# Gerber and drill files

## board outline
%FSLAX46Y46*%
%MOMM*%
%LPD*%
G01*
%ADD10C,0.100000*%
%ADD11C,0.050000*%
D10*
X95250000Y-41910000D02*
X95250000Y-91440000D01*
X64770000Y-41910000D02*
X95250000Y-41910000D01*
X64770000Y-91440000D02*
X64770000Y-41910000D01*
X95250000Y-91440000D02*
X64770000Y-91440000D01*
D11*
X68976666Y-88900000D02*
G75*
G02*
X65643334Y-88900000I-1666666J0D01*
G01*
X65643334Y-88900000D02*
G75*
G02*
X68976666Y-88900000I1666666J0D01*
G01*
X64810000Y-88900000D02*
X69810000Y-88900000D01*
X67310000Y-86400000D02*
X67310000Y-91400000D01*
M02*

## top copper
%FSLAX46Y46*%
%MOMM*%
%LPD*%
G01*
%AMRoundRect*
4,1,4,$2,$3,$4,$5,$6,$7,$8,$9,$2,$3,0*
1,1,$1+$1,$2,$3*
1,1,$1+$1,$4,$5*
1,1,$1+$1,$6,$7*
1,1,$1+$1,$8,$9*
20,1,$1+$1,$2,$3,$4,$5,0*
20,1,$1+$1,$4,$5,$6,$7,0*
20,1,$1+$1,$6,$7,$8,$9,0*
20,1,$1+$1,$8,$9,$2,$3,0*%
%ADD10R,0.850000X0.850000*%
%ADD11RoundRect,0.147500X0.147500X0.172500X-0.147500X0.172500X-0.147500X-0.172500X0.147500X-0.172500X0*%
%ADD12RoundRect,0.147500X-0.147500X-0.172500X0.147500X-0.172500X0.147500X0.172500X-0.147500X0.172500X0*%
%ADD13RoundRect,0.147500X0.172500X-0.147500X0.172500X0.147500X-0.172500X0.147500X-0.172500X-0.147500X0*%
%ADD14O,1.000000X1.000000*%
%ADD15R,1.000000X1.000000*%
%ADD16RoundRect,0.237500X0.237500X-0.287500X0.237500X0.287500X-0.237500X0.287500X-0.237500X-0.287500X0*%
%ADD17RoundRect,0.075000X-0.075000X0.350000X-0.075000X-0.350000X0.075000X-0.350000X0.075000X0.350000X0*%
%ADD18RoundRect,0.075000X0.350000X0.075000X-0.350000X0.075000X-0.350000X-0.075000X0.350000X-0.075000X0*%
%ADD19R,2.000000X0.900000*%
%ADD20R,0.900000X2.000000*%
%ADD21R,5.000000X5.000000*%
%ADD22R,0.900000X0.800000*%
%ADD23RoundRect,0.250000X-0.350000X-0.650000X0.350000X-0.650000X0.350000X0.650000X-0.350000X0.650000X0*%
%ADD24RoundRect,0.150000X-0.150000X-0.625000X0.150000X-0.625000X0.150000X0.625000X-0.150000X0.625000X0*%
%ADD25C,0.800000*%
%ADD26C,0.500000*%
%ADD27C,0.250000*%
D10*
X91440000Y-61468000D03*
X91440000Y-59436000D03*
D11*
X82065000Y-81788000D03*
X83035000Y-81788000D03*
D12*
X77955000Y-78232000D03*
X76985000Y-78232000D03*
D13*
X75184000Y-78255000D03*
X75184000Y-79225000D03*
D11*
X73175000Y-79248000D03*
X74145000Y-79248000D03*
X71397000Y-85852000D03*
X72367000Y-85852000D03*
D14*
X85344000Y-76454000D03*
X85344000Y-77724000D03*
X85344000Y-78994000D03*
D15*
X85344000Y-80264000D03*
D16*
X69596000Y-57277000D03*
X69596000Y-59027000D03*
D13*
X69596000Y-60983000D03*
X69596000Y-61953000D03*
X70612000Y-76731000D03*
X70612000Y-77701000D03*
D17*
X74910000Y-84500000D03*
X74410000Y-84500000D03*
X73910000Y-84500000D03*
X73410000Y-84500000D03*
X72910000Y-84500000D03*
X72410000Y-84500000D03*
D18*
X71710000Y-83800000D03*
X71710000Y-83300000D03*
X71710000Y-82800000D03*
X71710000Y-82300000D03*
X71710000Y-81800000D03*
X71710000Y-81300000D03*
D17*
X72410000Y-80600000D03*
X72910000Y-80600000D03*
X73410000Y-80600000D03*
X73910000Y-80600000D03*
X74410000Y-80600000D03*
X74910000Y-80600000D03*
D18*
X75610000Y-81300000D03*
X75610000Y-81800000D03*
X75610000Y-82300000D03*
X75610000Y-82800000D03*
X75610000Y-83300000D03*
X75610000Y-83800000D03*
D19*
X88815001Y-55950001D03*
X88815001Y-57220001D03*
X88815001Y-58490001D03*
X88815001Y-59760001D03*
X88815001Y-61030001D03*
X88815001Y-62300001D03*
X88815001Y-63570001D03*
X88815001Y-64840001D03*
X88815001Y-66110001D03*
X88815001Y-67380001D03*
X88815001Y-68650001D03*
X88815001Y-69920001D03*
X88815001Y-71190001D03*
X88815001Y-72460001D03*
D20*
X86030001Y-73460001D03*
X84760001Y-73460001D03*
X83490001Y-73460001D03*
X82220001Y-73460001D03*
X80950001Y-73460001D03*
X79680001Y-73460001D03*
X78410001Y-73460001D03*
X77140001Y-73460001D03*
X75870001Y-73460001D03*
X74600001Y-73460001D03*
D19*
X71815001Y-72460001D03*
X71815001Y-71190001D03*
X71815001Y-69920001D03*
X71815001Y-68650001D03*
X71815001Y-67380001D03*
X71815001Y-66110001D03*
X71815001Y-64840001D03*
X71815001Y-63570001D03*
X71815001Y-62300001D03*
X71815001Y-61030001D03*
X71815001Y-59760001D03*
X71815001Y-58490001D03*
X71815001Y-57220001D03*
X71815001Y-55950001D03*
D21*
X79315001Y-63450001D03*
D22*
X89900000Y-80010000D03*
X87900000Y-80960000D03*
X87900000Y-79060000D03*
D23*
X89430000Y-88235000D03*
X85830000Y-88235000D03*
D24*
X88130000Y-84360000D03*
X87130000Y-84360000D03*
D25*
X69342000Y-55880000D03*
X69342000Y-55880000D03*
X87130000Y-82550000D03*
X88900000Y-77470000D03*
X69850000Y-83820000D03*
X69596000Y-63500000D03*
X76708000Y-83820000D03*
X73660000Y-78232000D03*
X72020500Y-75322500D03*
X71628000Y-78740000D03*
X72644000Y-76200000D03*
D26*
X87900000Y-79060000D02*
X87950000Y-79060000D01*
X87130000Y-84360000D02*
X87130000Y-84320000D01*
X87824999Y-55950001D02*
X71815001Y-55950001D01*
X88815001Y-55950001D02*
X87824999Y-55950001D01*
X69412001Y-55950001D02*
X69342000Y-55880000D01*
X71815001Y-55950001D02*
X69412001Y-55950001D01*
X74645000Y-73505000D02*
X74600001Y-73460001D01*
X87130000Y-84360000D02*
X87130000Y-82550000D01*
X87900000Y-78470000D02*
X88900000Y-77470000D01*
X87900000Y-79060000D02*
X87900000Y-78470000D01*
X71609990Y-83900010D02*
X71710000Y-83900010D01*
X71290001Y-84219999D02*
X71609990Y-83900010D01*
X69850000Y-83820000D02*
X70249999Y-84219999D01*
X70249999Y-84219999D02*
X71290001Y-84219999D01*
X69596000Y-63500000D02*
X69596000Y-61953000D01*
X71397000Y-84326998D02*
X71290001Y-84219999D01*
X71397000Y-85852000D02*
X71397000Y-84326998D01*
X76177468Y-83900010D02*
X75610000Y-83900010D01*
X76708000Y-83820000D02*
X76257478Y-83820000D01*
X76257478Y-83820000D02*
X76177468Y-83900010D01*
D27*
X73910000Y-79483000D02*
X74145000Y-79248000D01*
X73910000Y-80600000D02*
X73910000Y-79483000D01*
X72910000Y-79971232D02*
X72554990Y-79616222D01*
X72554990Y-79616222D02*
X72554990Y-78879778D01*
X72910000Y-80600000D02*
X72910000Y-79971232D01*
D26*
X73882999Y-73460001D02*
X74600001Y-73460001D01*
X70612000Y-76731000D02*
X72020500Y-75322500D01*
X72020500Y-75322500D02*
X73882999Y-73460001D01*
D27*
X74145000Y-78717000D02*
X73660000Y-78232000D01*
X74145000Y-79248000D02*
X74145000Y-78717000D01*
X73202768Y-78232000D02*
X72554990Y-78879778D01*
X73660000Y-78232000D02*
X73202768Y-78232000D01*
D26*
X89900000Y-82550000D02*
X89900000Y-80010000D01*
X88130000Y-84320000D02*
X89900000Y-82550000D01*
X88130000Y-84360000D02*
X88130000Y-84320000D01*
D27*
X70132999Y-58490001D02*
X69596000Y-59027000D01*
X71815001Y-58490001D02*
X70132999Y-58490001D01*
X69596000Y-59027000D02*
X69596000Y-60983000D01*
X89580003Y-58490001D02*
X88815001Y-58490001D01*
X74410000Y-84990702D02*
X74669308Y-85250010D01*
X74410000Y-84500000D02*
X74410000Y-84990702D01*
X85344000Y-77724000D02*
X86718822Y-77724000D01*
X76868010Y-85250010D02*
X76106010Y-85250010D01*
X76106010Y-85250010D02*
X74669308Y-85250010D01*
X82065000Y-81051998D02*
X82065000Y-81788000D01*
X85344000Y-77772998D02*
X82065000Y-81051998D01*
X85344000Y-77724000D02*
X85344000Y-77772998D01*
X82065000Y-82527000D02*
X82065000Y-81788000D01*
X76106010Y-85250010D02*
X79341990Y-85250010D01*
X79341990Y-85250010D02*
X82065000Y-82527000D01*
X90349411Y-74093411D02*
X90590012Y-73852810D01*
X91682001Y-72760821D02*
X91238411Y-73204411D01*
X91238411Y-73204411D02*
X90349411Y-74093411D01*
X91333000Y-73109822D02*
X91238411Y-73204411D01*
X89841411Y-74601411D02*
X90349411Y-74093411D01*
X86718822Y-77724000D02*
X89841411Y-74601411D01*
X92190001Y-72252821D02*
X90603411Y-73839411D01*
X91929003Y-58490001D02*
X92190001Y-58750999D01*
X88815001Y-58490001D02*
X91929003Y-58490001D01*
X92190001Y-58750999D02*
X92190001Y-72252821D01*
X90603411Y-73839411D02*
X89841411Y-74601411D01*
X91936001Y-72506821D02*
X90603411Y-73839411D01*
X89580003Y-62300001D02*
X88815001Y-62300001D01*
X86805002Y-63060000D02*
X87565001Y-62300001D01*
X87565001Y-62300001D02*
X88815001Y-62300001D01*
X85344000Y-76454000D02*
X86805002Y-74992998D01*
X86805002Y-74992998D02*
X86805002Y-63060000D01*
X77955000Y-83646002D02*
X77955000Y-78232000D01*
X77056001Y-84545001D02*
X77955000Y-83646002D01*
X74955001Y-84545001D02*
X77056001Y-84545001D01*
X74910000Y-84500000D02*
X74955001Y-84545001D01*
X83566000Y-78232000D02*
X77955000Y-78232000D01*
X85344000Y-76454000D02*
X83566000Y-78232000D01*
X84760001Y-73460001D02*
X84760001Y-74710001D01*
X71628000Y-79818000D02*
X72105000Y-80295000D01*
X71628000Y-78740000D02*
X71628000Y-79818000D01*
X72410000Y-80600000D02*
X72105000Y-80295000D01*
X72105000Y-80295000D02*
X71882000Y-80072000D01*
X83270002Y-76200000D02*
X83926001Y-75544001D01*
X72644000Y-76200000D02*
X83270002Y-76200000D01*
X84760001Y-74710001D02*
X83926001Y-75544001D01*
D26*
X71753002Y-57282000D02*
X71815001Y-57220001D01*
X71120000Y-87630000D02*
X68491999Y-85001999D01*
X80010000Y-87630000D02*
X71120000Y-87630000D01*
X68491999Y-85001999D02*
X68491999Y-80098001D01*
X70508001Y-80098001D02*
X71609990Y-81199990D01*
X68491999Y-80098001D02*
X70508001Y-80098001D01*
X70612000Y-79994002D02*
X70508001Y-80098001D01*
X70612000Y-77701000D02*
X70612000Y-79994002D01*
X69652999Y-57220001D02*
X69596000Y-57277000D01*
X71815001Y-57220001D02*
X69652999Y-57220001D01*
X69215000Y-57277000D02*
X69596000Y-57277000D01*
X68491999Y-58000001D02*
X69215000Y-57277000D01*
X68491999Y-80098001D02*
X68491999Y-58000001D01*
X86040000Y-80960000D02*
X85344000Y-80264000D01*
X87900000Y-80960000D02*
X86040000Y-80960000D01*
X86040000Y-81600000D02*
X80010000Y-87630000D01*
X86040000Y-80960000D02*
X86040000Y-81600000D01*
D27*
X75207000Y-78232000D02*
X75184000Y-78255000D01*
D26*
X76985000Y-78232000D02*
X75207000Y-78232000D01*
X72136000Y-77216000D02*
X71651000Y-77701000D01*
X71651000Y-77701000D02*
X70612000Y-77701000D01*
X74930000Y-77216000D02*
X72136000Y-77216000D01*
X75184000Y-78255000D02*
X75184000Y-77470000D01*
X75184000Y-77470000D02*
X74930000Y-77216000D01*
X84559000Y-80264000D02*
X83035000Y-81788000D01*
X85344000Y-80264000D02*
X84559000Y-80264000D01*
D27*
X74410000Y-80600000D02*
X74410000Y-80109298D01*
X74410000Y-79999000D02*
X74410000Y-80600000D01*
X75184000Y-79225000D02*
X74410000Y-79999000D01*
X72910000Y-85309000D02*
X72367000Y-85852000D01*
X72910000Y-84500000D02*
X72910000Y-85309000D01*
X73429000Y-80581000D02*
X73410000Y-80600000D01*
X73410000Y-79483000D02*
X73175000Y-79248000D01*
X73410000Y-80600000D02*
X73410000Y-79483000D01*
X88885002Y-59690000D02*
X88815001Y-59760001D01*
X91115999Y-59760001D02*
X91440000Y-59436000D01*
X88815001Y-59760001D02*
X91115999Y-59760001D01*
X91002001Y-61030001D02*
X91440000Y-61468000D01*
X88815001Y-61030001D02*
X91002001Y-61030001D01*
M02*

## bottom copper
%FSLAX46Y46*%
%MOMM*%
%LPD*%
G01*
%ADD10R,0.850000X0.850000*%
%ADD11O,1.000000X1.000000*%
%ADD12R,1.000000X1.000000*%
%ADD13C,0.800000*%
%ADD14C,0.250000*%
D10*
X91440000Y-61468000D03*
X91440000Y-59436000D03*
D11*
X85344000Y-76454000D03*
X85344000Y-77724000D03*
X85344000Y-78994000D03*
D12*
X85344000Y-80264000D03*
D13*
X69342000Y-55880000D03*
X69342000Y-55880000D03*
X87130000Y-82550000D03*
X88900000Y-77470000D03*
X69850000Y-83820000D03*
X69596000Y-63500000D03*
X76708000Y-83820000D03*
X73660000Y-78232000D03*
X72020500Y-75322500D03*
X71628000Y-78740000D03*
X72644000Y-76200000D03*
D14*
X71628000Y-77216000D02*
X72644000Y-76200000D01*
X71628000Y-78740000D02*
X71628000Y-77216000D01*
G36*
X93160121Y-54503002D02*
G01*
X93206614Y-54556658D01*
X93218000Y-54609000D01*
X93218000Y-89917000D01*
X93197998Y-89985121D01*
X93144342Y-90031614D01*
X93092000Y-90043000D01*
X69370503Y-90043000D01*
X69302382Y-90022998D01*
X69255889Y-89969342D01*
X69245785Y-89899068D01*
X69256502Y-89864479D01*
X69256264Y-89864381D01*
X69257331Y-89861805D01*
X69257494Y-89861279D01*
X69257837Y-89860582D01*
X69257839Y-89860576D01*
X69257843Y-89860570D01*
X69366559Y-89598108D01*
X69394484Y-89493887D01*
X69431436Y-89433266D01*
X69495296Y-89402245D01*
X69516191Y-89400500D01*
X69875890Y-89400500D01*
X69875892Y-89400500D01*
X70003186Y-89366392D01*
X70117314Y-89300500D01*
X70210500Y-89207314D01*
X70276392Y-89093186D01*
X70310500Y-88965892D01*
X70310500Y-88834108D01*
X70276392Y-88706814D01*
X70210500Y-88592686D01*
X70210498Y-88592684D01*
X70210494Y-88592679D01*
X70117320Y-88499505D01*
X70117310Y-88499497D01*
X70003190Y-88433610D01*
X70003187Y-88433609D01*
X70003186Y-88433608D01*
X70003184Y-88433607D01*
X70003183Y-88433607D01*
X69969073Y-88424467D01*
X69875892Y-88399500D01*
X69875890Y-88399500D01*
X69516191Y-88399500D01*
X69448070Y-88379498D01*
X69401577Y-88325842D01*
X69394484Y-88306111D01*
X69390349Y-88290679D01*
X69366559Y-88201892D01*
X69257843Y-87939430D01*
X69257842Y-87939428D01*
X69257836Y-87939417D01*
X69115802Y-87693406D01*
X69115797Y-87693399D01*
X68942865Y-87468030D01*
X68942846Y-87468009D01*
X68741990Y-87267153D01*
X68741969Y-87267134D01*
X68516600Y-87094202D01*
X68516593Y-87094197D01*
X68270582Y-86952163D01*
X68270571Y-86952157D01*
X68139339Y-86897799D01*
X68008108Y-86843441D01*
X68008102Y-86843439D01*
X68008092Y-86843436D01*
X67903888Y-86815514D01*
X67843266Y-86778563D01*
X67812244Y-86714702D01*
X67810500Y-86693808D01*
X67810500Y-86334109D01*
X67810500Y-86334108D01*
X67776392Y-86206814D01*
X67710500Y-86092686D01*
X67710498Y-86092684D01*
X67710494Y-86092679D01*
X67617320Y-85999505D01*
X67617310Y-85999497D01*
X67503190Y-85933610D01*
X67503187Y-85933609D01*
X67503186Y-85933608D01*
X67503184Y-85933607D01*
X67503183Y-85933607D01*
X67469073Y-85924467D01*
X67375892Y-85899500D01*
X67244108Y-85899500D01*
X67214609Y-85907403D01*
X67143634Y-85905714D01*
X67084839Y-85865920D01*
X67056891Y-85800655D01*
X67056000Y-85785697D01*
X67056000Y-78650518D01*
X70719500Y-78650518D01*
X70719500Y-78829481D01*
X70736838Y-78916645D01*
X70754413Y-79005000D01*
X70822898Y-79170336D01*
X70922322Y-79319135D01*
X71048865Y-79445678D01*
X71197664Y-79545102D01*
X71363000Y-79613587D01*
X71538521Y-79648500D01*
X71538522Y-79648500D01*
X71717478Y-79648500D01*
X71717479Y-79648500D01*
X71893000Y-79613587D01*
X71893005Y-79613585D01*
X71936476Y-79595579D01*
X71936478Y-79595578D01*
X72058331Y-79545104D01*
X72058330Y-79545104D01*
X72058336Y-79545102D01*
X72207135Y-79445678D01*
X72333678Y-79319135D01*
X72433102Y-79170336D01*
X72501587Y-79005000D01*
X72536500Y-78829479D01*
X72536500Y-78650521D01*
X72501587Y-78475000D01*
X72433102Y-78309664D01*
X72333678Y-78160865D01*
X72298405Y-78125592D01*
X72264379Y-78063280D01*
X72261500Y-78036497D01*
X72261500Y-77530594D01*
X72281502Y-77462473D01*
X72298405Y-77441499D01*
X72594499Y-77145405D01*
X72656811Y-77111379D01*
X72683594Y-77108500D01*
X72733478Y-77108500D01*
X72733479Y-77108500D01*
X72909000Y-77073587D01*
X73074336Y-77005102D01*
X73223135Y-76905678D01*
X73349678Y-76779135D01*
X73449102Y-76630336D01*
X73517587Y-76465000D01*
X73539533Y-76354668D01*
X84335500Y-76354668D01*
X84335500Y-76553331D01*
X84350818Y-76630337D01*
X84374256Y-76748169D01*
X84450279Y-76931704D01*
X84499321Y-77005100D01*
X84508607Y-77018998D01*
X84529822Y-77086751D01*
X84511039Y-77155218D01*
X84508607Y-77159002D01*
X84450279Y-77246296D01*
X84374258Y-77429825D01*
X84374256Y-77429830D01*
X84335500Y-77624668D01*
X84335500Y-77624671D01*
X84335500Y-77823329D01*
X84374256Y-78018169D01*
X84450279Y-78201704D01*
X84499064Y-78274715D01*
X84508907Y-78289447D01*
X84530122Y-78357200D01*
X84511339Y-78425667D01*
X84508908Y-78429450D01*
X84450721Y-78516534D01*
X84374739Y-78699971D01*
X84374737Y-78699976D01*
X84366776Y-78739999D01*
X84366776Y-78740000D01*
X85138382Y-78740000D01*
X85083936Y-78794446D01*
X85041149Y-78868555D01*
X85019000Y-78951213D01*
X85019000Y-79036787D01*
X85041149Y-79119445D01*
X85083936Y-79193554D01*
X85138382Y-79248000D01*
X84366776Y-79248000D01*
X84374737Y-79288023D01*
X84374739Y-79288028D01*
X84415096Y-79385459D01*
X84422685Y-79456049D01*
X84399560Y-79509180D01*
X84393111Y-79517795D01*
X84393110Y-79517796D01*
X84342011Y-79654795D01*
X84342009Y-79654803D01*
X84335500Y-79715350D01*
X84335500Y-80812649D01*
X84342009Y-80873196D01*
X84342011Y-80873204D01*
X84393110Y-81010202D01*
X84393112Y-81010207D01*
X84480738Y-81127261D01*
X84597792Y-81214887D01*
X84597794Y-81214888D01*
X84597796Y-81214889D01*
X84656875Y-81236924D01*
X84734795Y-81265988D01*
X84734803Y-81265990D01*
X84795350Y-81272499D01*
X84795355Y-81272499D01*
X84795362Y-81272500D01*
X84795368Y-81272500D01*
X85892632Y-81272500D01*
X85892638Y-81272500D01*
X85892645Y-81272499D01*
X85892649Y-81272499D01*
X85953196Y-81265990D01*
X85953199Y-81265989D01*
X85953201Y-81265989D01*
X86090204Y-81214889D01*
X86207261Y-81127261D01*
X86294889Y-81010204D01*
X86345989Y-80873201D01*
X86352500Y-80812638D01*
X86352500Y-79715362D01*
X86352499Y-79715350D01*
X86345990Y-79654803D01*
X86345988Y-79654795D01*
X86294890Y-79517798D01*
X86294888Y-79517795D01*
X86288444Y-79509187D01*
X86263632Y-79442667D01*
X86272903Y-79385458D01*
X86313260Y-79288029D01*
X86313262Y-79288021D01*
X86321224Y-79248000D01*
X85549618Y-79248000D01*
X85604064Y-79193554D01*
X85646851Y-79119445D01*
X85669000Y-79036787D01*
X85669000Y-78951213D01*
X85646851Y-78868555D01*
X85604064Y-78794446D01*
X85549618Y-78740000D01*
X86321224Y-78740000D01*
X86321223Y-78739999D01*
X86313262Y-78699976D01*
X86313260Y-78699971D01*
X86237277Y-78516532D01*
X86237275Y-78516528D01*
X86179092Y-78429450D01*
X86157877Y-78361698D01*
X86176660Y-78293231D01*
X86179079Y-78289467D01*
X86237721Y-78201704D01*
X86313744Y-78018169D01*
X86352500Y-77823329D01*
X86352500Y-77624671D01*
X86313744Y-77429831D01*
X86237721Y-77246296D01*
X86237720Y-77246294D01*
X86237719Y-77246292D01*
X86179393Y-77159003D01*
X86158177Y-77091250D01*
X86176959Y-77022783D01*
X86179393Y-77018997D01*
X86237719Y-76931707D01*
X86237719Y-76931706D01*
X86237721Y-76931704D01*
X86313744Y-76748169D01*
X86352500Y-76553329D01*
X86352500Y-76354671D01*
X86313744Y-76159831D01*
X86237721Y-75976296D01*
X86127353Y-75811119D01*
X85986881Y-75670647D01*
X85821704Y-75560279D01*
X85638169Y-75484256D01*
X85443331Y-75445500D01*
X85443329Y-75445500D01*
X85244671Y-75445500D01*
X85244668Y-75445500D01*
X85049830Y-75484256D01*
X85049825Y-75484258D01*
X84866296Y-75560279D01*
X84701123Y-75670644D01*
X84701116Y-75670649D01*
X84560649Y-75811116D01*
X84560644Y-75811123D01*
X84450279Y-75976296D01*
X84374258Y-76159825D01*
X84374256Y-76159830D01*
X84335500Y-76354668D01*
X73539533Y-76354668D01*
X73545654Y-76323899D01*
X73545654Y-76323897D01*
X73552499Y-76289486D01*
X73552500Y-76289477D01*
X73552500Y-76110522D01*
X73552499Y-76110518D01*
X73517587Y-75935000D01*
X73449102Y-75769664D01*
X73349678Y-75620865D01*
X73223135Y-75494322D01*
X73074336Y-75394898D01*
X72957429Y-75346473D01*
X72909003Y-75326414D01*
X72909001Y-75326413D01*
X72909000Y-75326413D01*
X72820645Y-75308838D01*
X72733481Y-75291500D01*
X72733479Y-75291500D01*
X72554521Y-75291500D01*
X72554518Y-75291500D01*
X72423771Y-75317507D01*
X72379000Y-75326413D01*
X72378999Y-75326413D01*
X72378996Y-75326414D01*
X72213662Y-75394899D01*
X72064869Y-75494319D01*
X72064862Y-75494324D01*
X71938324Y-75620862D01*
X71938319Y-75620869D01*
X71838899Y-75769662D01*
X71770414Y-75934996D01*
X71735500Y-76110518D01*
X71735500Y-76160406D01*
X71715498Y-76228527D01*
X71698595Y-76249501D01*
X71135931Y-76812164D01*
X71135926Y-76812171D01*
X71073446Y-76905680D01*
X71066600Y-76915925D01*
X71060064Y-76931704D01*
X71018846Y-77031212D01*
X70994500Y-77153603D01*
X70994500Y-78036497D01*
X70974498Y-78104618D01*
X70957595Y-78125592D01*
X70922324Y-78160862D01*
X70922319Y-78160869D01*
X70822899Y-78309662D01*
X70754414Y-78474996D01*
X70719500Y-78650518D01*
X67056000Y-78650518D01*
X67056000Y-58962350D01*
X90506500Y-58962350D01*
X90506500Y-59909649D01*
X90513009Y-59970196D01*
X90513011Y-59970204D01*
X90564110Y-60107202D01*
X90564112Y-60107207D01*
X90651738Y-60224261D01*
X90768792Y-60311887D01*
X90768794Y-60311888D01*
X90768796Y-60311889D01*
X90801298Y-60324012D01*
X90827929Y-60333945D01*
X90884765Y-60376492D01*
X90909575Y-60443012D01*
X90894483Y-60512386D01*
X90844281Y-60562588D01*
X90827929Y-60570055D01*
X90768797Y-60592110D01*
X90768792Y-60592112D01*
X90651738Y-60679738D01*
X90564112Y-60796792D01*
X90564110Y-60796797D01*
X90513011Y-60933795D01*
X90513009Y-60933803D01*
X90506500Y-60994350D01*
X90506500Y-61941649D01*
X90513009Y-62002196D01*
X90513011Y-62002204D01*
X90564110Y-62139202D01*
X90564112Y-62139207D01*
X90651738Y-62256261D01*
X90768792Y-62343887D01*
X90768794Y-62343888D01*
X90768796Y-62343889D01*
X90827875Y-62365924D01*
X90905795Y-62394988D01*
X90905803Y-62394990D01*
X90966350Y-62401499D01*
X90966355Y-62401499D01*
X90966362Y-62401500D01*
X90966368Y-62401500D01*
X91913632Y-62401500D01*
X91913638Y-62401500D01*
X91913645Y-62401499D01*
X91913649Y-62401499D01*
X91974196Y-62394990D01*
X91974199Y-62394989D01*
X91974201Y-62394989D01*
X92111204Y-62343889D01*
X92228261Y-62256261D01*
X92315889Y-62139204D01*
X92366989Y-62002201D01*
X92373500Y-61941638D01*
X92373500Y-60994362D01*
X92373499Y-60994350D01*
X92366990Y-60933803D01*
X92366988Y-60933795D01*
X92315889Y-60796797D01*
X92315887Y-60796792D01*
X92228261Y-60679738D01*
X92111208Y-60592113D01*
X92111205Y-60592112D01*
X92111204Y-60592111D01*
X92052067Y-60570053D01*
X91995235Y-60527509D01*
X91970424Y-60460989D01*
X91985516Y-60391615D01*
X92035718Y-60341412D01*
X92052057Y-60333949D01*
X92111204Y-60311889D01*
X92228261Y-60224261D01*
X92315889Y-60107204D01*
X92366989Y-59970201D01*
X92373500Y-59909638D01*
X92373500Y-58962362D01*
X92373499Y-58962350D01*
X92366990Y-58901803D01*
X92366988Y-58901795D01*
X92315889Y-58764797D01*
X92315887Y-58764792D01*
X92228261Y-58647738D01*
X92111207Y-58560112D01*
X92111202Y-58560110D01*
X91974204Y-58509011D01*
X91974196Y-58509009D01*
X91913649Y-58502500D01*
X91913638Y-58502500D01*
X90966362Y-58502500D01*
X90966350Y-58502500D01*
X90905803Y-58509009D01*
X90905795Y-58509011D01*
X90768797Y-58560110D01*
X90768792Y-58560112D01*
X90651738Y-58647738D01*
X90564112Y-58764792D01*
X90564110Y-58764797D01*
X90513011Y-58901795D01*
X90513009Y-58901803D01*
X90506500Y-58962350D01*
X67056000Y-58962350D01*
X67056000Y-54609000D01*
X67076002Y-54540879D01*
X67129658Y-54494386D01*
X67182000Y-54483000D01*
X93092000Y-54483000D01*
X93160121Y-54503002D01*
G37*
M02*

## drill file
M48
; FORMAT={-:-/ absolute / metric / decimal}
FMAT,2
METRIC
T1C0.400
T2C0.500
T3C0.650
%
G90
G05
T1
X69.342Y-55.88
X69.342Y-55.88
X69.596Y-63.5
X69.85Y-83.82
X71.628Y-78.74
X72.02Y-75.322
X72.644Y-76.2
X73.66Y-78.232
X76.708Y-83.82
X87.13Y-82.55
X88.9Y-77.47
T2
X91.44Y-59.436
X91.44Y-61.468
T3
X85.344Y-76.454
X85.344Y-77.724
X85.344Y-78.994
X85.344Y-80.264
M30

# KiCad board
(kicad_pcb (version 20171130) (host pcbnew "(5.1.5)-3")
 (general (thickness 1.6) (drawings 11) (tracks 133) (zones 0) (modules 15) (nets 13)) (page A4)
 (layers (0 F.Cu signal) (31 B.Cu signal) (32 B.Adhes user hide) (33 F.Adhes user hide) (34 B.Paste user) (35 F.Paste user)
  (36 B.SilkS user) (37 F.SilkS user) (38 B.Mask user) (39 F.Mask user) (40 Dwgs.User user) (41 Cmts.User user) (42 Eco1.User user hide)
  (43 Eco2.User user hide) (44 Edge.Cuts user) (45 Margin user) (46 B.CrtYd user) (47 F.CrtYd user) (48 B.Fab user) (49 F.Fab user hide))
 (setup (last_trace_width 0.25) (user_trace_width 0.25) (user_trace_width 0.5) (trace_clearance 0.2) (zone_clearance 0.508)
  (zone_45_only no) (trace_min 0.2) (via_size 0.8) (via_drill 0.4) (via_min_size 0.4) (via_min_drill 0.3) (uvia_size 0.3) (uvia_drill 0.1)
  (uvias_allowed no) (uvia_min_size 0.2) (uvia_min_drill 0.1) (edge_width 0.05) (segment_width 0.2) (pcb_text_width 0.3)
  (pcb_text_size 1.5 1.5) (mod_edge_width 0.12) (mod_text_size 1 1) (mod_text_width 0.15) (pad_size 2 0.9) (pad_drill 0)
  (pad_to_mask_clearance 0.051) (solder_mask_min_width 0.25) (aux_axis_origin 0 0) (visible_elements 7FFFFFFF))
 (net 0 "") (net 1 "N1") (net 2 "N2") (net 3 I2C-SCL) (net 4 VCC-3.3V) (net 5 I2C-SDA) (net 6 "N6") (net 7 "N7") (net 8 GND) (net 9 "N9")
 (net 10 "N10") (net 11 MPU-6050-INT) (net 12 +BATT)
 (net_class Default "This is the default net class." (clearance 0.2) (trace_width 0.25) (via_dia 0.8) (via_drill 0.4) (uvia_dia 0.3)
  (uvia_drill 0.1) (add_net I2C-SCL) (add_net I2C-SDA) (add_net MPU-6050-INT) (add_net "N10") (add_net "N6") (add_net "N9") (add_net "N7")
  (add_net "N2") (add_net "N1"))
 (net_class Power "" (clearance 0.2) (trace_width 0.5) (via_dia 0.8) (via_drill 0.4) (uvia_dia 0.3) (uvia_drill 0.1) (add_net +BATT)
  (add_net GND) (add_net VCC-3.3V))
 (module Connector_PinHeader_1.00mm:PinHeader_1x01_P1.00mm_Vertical (layer F.Cu) (at 91.44 61.468)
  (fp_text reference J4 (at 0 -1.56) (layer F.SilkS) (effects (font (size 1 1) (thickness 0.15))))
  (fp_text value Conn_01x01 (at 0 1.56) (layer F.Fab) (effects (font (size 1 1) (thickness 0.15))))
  (pad 1 thru_hole rect (at 0 0) (size 0.85 0.85) (drill 0.5) (layers *.Cu *.Mask) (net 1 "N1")))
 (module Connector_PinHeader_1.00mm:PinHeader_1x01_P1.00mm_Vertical (layer F.Cu) (at 91.44 59.436)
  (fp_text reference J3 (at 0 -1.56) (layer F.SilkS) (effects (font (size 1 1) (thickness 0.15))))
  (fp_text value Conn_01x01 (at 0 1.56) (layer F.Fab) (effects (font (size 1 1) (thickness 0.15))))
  (pad 1 thru_hole rect (at 0 0) (size 0.85 0.85) (drill 0.5) (layers *.Cu *.Mask) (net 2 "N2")))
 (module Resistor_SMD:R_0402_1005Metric (layer F.Cu) (at 82.55 81.788 180)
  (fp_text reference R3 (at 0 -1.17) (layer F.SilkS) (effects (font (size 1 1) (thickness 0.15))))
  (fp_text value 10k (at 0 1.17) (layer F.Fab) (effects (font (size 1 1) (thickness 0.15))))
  (pad 2 smd roundrect (at 0.485 0 180) (size 0.59 0.64) (layers F.Cu F.Paste F.Mask) (roundrect_rratio 0.25) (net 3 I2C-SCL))
  (pad 1 smd roundrect (at -0.485 0 180) (size 0.59 0.64) (layers F.Cu F.Paste F.Mask) (roundrect_rratio 0.25) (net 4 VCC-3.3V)))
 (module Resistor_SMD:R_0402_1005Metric (layer F.Cu) (at 77.47 78.232)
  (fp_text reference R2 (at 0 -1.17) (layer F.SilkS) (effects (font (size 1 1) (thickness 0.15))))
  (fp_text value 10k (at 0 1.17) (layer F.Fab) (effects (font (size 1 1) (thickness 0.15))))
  (pad 2 smd roundrect (at 0.485 0) (size 0.59 0.64) (layers F.Cu F.Paste F.Mask) (roundrect_rratio 0.25) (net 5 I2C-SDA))
  (pad 1 smd roundrect (at -0.485 0) (size 0.59 0.64) (layers F.Cu F.Paste F.Mask) (roundrect_rratio 0.25) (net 4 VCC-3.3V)))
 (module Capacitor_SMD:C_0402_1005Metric (layer F.Cu) (at 75.184 78.74 90)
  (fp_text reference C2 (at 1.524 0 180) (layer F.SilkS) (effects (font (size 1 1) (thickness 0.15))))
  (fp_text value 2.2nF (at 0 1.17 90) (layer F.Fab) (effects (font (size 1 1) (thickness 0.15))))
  (pad 2 smd roundrect (at 0.485 0 90) (size 0.59 0.64) (layers F.Cu F.Paste F.Mask) (roundrect_rratio 0.25) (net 4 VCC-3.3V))
  (pad 1 smd roundrect (at -0.485 0 90) (size 0.59 0.64) (layers F.Cu F.Paste F.Mask) (roundrect_rratio 0.25) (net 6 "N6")))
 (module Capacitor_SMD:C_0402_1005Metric (layer F.Cu) (at 73.66 79.248 180)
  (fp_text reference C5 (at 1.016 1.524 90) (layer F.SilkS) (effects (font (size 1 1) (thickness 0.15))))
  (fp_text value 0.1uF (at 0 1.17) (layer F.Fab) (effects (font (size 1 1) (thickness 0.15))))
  (pad 2 smd roundrect (at 0.485 0 180) (size 0.59 0.64) (layers F.Cu F.Paste F.Mask) (roundrect_rratio 0.25) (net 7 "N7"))
  (pad 1 smd roundrect (at -0.485 0 180) (size 0.59 0.64) (layers F.Cu F.Paste F.Mask) (roundrect_rratio 0.25) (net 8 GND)))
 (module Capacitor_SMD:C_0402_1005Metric (layer F.Cu) (at 71.882 85.852 180)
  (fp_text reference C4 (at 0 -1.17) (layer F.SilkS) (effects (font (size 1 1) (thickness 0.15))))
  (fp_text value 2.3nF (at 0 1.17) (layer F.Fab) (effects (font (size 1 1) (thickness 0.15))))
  (pad 2 smd roundrect (at 0.485 0 180) (size 0.59 0.64) (layers F.Cu F.Paste F.Mask) (roundrect_rratio 0.25) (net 8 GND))
  (pad 1 smd roundrect (at -0.485 0 180) (size 0.59 0.64) (layers F.Cu F.Paste F.Mask) (roundrect_rratio 0.25) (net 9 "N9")))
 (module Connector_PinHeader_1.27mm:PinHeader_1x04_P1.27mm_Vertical (layer F.Cu) (at 85.344 80.264 180)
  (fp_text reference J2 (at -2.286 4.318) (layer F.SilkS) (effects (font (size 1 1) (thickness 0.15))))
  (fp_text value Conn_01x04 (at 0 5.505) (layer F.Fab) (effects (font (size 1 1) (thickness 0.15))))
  (pad 4 thru_hole oval (at 0 3.81 180) (size 1 1) (drill 0.65) (layers *.Cu *.Mask) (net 5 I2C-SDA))
  (pad 3 thru_hole oval (at 0 2.54 180) (size 1 1) (drill 0.65) (layers *.Cu *.Mask) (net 3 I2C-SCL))
  (pad 2 thru_hole oval (at 0 1.27 180) (size 1 1) (drill 0.65) (layers *.Cu *.Mask) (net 8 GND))
  (pad 1 thru_hole rect (at 0 0 180) (size 1 1) (drill 0.65) (layers *.Cu *.Mask) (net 4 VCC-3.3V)))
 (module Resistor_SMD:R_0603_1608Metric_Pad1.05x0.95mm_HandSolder (layer F.Cu) (at 69.596 58.152 90)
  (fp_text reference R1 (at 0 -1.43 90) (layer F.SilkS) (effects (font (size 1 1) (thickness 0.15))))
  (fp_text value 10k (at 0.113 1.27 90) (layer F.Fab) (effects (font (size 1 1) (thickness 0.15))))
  (pad 2 smd roundrect (at 0.875 0 90) (size 1.05 0.95) (layers F.Cu F.Paste F.Mask) (roundrect_rratio 0.25) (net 4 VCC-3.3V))
  (pad 1 smd roundrect (at -0.875 0 90) (size 1.05 0.95) (layers F.Cu F.Paste F.Mask) (roundrect_rratio 0.25) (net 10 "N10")))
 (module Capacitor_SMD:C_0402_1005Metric (layer F.Cu) (at 69.596 61.468 90)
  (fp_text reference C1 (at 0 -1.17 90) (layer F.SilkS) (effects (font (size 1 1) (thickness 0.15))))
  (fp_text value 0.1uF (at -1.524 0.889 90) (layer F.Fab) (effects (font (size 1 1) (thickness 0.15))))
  (pad 2 smd roundrect (at 0.485 0 90) (size 0.59 0.64) (layers F.Cu F.Paste F.Mask) (roundrect_rratio 0.25) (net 10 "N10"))
  (pad 1 smd roundrect (at -0.485 0 90) (size 0.59 0.64) (layers F.Cu F.Paste F.Mask) (roundrect_rratio 0.25) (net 8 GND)))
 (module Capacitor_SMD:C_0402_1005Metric (layer F.Cu) (at 70.612 77.216 90)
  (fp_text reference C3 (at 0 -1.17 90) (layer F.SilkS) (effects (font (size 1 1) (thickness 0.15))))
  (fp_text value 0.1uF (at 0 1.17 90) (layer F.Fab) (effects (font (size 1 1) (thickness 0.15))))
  (pad 2 smd roundrect (at 0.485 0 90) (size 0.59 0.64) (layers F.Cu F.Paste F.Mask) (roundrect_rratio 0.25) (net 8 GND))
  (pad 1 smd roundrect (at -0.485 0 90) (size 0.59 0.64) (layers F.Cu F.Paste F.Mask) (roundrect_rratio 0.25) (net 4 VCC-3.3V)))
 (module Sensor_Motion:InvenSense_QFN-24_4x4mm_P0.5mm (layer F.Cu) (at 73.66 82.55 180)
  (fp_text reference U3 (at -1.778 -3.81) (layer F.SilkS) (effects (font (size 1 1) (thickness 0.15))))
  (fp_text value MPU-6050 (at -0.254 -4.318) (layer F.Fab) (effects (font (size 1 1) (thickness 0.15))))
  (pad 24 smd roundrect (at -1.25 -1.95 270) (size 0.85 0.3) (layers F.Cu F.Paste F.Mask) (roundrect_rratio 0.25) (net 5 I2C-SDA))
  (pad 23 smd roundrect (at -0.75 -1.95 270) (size 0.85 0.3) (layers F.Cu F.Paste F.Mask) (roundrect_rratio 0.25) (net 3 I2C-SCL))
  (pad 22 smd roundrect (at -0.25 -1.95 270) (size 0.85 0.3) (layers F.Cu F.Paste F.Mask) (roundrect_rratio 0.25))
  (pad 21 smd roundrect (at 0.25 -1.95 270) (size 0.85 0.3) (layers F.Cu F.Paste F.Mask) (roundrect_rratio 0.25))
  (pad 20 smd roundrect (at 0.75 -1.95 270) (size 0.85 0.3) (layers F.Cu F.Paste F.Mask) (roundrect_rratio 0.25) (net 9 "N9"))
  (pad 19 smd roundrect (at 1.25 -1.95 270) (size 0.85 0.3) (layers F.Cu F.Paste F.Mask) (roundrect_rratio 0.25))
  (pad 18 smd roundrect (at 1.95 -1.25 180) (size 0.85 0.3) (layers F.Cu F.Paste F.Mask) (roundrect_rratio 0.25) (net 8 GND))
  (pad 17 smd roundrect (at 1.95 -0.75 180) (size 0.85 0.3) (layers F.Cu F.Paste F.Mask) (roundrect_rratio 0.25))
  (pad 16 smd roundrect (at 1.95 -0.25 180) (size 0.85 0.3) (layers F.Cu F.Paste F.Mask) (roundrect_rratio 0.25))
  (pad 15 smd roundrect (at 1.95 0.25 180) (size 0.85 0.3) (layers F.Cu F.Paste F.Mask) (roundrect_rratio 0.25))
  (pad 14 smd roundrect (at 1.95 0.75 180) (size 0.85 0.3) (layers F.Cu F.Paste F.Mask) (roundrect_rratio 0.25))
  (pad 13 smd roundrect (at 1.95 1.25 180) (size 0.85 0.3) (layers F.Cu F.Paste F.Mask) (roundrect_rratio 0.25) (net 4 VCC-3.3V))
  (pad 12 smd roundrect (at 1.25 1.95 270) (size 0.85 0.3) (layers F.Cu F.Paste F.Mask) (roundrect_rratio 0.25) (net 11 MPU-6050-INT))
  (pad 11 smd roundrect (at 0.75 1.95 270) (size 0.85 0.3) (layers F.Cu F.Paste F.Mask) (roundrect_rratio 0.25) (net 8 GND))
  (pad 10 smd roundrect (at 0.25 1.95 270) (size 0.85 0.3) (layers F.Cu F.Paste F.Mask) (roundrect_rratio 0.25) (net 7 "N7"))
  (pad 9 smd roundrect (at -0.25 1.95 270) (size 0.85 0.3) (layers F.Cu F.Paste F.Mask) (roundrect_rratio 0.25) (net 8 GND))
  (pad 8 smd roundrect (at -0.75 1.95 270) (size 0.85 0.3) (layers F.Cu F.Paste F.Mask) (roundrect_rratio 0.25) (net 6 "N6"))
  (pad 7 smd roundrect (at -1.25 1.95 270) (size 0.85 0.3) (layers F.Cu F.Paste F.Mask) (roundrect_rratio 0.25))
  (pad 6 smd roundrect (at -1.95 1.25 180) (size 0.85 0.3) (layers F.Cu F.Paste F.Mask) (roundrect_rratio 0.25))
  (pad 5 smd roundrect (at -1.95 0.75 180) (size 0.85 0.3) (layers F.Cu F.Paste F.Mask) (roundrect_rratio 0.25))
  (pad 4 smd roundrect (at -1.95 0.25 180) (size 0.85 0.3) (layers F.Cu F.Paste F.Mask) (roundrect_rratio 0.25))
  (pad 3 smd roundrect (at -1.95 -0.25 180) (size 0.85 0.3) (layers F.Cu F.Paste F.Mask) (roundrect_rratio 0.25))
  (pad 2 smd roundrect (at -1.95 -0.75 180) (size 0.85 0.3) (layers F.Cu F.Paste F.Mask) (roundrect_rratio 0.25))
  (pad 1 smd roundrect (at -1.95 -1.25 180) (size 0.85 0.3) (layers F.Cu F.Paste F.Mask) (roundrect_rratio 0.25) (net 8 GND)))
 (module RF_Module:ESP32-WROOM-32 (layer F.Cu) (at 80.315001 64.205001)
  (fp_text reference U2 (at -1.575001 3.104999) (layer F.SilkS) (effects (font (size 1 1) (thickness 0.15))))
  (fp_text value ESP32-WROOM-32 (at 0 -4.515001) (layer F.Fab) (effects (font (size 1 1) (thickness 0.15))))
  (pad 38 smd rect (at 8.5 -8.255) (size 2 0.9) (layers F.Cu F.Paste F.Mask) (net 8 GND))
  (pad 37 smd rect (at 8.5 -6.985) (size 2 0.9) (layers F.Cu F.Paste F.Mask))
  (pad 36 smd rect (at 8.5 -5.715) (size 2 0.9) (layers F.Cu F.Paste F.Mask) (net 3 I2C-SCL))
  (pad 35 smd rect (at 8.5 -4.445) (size 2 0.9) (layers F.Cu F.Paste F.Mask) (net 2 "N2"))
  (pad 34 smd rect (at 8.5 -3.175) (size 2 0.9) (layers F.Cu F.Paste F.Mask) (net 1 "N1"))
  (pad 33 smd rect (at 8.5 -1.905) (size 2 0.9) (layers F.Cu F.Paste F.Mask) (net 5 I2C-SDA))
  (pad 32 smd rect (at 8.5 -0.635) (size 2 0.9) (layers F.Cu F.Paste F.Mask))
  (pad 31 smd rect (at 8.5 0.635) (size 2 0.9) (layers F.Cu F.Paste F.Mask))
  (pad 30 smd rect (at 8.5 1.905) (size 2 0.9) (layers F.Cu F.Paste F.Mask))
  (pad 29 smd rect (at 8.5 3.175) (size 2 0.9) (layers F.Cu F.Paste F.Mask))
  (pad 28 smd rect (at 8.5 4.445) (size 2 0.9) (layers F.Cu F.Paste F.Mask))
  (pad 27 smd rect (at 8.5 5.715) (size 2 0.9) (layers F.Cu F.Paste F.Mask))
  (pad 26 smd rect (at 8.5 6.985) (size 2 0.9) (layers F.Cu F.Paste F.Mask))
  (pad 25 smd rect (at 8.5 8.255) (size 2 0.9) (layers F.Cu F.Paste F.Mask))
  (pad 24 smd rect (at 5.715 9.255 90) (size 2 0.9) (layers F.Cu F.Paste F.Mask))
  (pad 23 smd rect (at 4.445 9.255 90) (size 2 0.9) (layers F.Cu F.Paste F.Mask) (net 11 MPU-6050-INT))
  (pad 22 smd rect (at 3.175 9.255 90) (size 2 0.9) (layers F.Cu F.Paste F.Mask))
  (pad 21 smd rect (at 1.905 9.255 90) (size 2 0.9) (layers F.Cu F.Paste F.Mask))
  (pad 20 smd rect (at 0.635 9.255 90) (size 2 0.9) (layers F.Cu F.Paste F.Mask))
  (pad 19 smd rect (at -0.635 9.255 90) (size 2 0.9) (layers F.Cu F.Paste F.Mask))
  (pad 18 smd rect (at -1.905 9.255 90) (size 2 0.9) (layers F.Cu F.Paste F.Mask))
  (pad 17 smd rect (at -3.175 9.255 90) (size 2 0.9) (layers F.Cu F.Paste F.Mask))
  (pad 16 smd rect (at -4.445 9.255 90) (size 2 0.9) (layers F.Cu F.Paste F.Mask))
  (pad 15 smd rect (at -5.715 9.255 90) (size 2 0.9) (layers F.Cu F.Paste F.Mask) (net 8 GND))
  (pad 14 smd rect (at -8.5 8.255) (size 2 0.9) (layers F.Cu F.Paste F.Mask))
  (pad 13 smd rect (at -8.5 6.985) (size 2 0.9) (layers F.Cu F.Paste F.Mask))
  (pad 12 smd rect (at -8.5 5.715) (size 2 0.9) (layers F.Cu F.Paste F.Mask))
  (pad 11 smd rect (at -8.5 4.445) (size 2 0.9) (layers F.Cu F.Paste F.Mask))
  (pad 10 smd rect (at -8.5 3.175) (size 2 0.9) (layers F.Cu F.Paste F.Mask))
  (pad 9 smd rect (at -8.5 1.905) (size 2 0.9) (layers F.Cu F.Paste F.Mask))
  (pad 8 smd rect (at -8.5 0.635) (size 2 0.9) (layers F.Cu F.Paste F.Mask))
  (pad 7 smd rect (at -8.5 -0.635) (size 2 0.9) (layers F.Cu F.Paste F.Mask))
  (pad 6 smd rect (at -8.5 -1.905) (size 2 0.9) (layers F.Cu F.Paste F.Mask))
  (pad 5 smd rect (at -8.5 -3.175) (size 2 0.9) (layers F.Cu F.Paste F.Mask))
  (pad 4 smd rect (at -8.5 -4.445) (size 2 0.9) (layers F.Cu F.Paste F.Mask))
  (pad 3 smd rect (at -8.5 -5.715) (size 2 0.9) (layers F.Cu F.Paste F.Mask) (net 10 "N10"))
  (pad 2 smd rect (at -8.5 -6.985) (size 2 0.9) (layers F.Cu F.Paste F.Mask) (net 4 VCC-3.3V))
  (pad 1 smd rect (at -8.5 -8.255) (size 2 0.9) (layers F.Cu F.Paste F.Mask) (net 8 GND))
  (pad 39 smd rect (at -1 -0.755) (size 5 5) (layers F.Cu F.Paste F.Mask) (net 8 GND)))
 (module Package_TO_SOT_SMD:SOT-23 (layer F.Cu) (at 88.9 80.01)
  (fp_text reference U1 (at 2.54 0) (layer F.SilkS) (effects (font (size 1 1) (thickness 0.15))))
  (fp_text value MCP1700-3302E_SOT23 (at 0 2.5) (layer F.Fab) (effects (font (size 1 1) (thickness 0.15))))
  (pad 3 smd rect (at 1 0) (size 0.9 0.8) (layers F.Cu F.Paste F.Mask) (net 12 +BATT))
  (pad 2 smd rect (at -1 0.95) (size 0.9 0.8) (layers F.Cu F.Paste F.Mask) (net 4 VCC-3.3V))
  (pad 1 smd rect (at -1 -0.95) (size 0.9 0.8) (layers F.Cu F.Paste F.Mask) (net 8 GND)))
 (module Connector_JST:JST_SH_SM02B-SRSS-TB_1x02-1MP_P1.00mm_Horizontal (layer F.Cu) (at 87.63 86.36)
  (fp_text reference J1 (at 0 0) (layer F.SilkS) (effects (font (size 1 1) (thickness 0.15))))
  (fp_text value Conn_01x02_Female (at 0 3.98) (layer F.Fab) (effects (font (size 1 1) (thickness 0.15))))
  (pad MP smd roundrect (at 1.8 1.875) (size 1.2 1.8) (layers F.Cu F.Paste F.Mask) (roundrect_rratio 0.208333))
  (pad MP smd roundrect (at -1.8 1.875) (size 1.2 1.8) (layers F.Cu F.Paste F.Mask) (roundrect_rratio 0.208333))
  (pad 2 smd roundrect (at 0.5 -2) (size 0.6 1.55) (layers F.Cu F.Paste F.Mask) (roundrect_rratio 0.25) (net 12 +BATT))
  (pad 1 smd roundrect (at -0.5 -2) (size 0.6 1.55) (layers F.Cu F.Paste F.Mask) (roundrect_rratio 0.25) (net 8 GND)))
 (gr_line (start 95.25 41.91) (end 95.25 91.44) (layer Edge.Cuts) (width 0.1))
 (gr_line (start 64.77 41.91) (end 95.25 41.91) (layer Edge.Cuts) (width 0.1))
 (gr_line (start 64.77 91.44) (end 64.77 41.91) (layer Edge.Cuts) (width 0.1))
 (gr_line (start 95.25 91.44) (end 64.77 91.44) (layer Edge.Cuts) (width 0.1))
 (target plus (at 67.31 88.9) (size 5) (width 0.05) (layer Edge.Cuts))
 (via (at 69.342 55.88) (size 0.8) (drill 0.4) (layers F.Cu B.Cu) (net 8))
 (via (at 69.342 55.88) (size 0.8) (drill 0.4) (layers F.Cu B.Cu) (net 8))
 (segment (start 87.9 79.06) (end 87.95 79.06) (width 0.5) (layer F.Cu) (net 8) (status 30))
 (segment (start 87.13 84.36) (end 87.13 84.32) (width 0.5) (layer F.Cu) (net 8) (status 30))
 (segment (start 87.824999 55.950001) (end 71.815001 55.950001) (width 0.5) (layer F.Cu) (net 8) (status 30))
 (segment (start 88.815001 55.950001) (end 87.824999 55.950001) (width 0.5) (layer F.Cu) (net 8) (status 30))
 (segment (start 69.412001 55.950001) (end 69.342 55.88) (width 0.5) (layer F.Cu) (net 8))
 (segment (start 71.815001 55.950001) (end 69.412001 55.950001) (width 0.5) (layer F.Cu) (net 8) (status 10))
 (segment (start 74.645 73.505) (end 74.600001 73.460001) (width 0.5) (layer F.Cu) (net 8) (status 30))
 (segment (start 87.13 84.36) (end 87.13 82.55) (width 0.5) (layer F.Cu) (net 8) (status 10))
 (via (at 87.13 82.55) (size 0.8) (drill 0.4) (layers F.Cu B.Cu) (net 8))
 (via (at 88.9 77.47) (size 0.8) (drill 0.4) (layers F.Cu B.Cu) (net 8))
 (segment (start 87.9 78.47) (end 88.9 77.47) (width 0.5) (layer F.Cu) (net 8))
 (segment (start 87.9 79.06) (end 87.9 78.47) (width 0.5) (layer F.Cu) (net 8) (status 10))
 (via (at 69.85 83.82) (size 0.8) (drill 0.4) (layers F.Cu B.Cu) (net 8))
 (segment (start 71.60999 83.90001) (end 71.71 83.90001) (width 0.5) (layer F.Cu) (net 8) (status 30))
 (segment (start 71.290001 84.219999) (end 71.60999 83.90001) (width 0.5) (layer F.Cu) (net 8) (status 20))
 (segment (start 69.85 83.82) (end 70.249999 84.219999) (width 0.5) (layer F.Cu) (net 8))
 (segment (start 70.249999 84.219999) (end 71.290001 84.219999) (width 0.5) (layer F.Cu) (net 8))
 (via (at 69.596 63.5) (size 0.8) (drill 0.4) (layers F.Cu B.Cu) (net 8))
 (segment (start 69.596 63.5) (end 69.596 61.953) (width 0.5) (layer F.Cu) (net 8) (status 20))
 (segment (start 71.397 84.326998) (end 71.290001 84.219999) (width 0.5) (layer F.Cu) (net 8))
 (segment (start 71.397 85.852) (end 71.397 84.326998) (width 0.5) (layer F.Cu) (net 8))
 (via (at 76.708 83.82) (size 0.8) (drill 0.4) (layers F.Cu B.Cu) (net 8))
 (segment (start 76.177468 83.90001) (end 75.61 83.90001) (width 0.5) (layer F.Cu) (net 8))
 (segment (start 76.708 83.82) (end 76.257478 83.82) (width 0.5) (layer F.Cu) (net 8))
 (segment (start 76.257478 83.82) (end 76.177468 83.90001) (width 0.5) (layer F.Cu) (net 8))
 (segment (start 73.91 79.483) (end 74.145 79.248) (width 0.25) (layer F.Cu) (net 8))
 (segment (start 73.91 80.6) (end 73.91 79.483) (width 0.25) (layer F.Cu) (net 8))
 (via (at 73.66 78.232) (size 0.8) (drill 0.4) (layers F.Cu B.Cu) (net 8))
 (segment (start 72.91 79.971232) (end 72.55499 79.616222) (width 0.25) (layer F.Cu) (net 8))
 (segment (start 72.55499 79.616222) (end 72.55499 78.879778) (width 0.25) (layer F.Cu) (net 8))
 (segment (start 72.91 80.6) (end 72.91 79.971232) (width 0.25) (layer F.Cu) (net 8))
 (segment (start 73.882999 73.460001) (end 74.600001 73.460001) (width 0.5) (layer F.Cu) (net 8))
 (segment (start 70.612 76.731) (end 72.0205 75.3225) (width 0.5) (layer F.Cu) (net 8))
 (segment (start 72.0205 75.3225) (end 73.882999 73.460001) (width 0.5) (layer F.Cu) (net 8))
 (via (at 72.0205 75.3225) (size 0.8) (drill 0.4) (layers F.Cu B.Cu) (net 8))
 (segment (start 74.145 78.717) (end 73.66 78.232) (width 0.25) (layer F.Cu) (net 8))
 (segment (start 74.145 79.248) (end 74.145 78.717) (width 0.25) (layer F.Cu) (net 8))
 (segment (start 73.202768 78.232) (end 72.55499 78.879778) (width 0.25) (layer F.Cu) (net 8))
 (segment (start 73.66 78.232) (end 73.202768 78.232) (width 0.25) (layer F.Cu) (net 8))
 (segment (start 89.9 82.55) (end 89.9 80.01) (width 0.5) (layer F.Cu) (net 12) (status 20))
 (segment (start 88.13 84.32) (end 89.9 82.55) (width 0.5) (layer F.Cu) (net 12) (status 10))
 (segment (start 88.13 84.36) (end 88.13 84.32) (width 0.5) (layer F.Cu) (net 12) (status 30))
 (segment (start 70.132999 58.490001) (end 69.596 59.027) (width 0.25) (layer F.Cu) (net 10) (status 20))
 (segment (start 71.815001 58.490001) (end 70.132999 58.490001) (width 0.25) (layer F.Cu) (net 10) (status 10))
 (segment (start 69.596 59.027) (end 69.596 60.983) (width 0.25) (layer F.Cu) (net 10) (status 30))
 (segment (start 89.580003 58.490001) (end 88.815001 58.490001) (width 0.25) (layer F.Cu) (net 3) (status 30))
 (segment (start 74.41 84.990702) (end 74.669308 85.25001) (width 0.25) (layer F.Cu) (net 3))
 (segment (start 74.41 84.5) (end 74.41 84.990702) (width 0.25) (layer F.Cu) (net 3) (status 10))
 (segment (start 85.344 77.724) (end 86.718822 77.724) (width 0.25) (layer F.Cu) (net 3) (status 10))
 (segment (start 76.86801 85.25001) (end 76.10601 85.25001) (width 0.25) (layer F.Cu) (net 3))
 (segment (start 76.10601 85.25001) (end 74.669308 85.25001) (width 0.25) (layer F.Cu) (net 3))
 (segment (start 82.065 81.051998) (end 82.065 81.788) (width 0.25) (layer F.Cu) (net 3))
 (segment (start 85.344 77.772998) (end 82.065 81.051998) (width 0.25) (layer F.Cu) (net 3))
 (segment (start 85.344 77.724) (end 85.344 77.772998) (width 0.25) (layer F.Cu) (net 3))
 (segment (start 82.065 82.527) (end 82.065 81.788) (width 0.25) (layer F.Cu) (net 3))
 (segment (start 76.10601 85.25001) (end 79.34199 85.25001) (width 0.25) (layer F.Cu) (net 3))
 (segment (start 79.34199 85.25001) (end 82.065 82.527) (width 0.25) (layer F.Cu) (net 3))
 (segment (start 90.349411 74.093411) (end 90.590012 73.85281) (width 0.25) (layer F.Cu) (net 3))
 (segment (start 91.682001 72.760821) (end 91.238411 73.204411) (width 0.25) (layer F.Cu) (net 3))
 (segment (start 91.238411 73.204411) (end 90.349411 74.093411) (width 0.25) (layer F.Cu) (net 3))
 (segment (start 91.333 73.109822) (end 91.238411 73.204411) (width 0.25) (layer F.Cu) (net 3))
 (segment (start 89.841411 74.601411) (end 90.349411 74.093411) (width 0.25) (layer F.Cu) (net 3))
 (segment (start 86.718822 77.724) (end 89.841411 74.601411) (width 0.25) (layer F.Cu) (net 3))
 (segment (start 92.190001 72.252821) (end 90.603411 73.839411) (width 0.25) (layer F.Cu) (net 3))
 (segment (start 91.929003 58.490001) (end 92.190001 58.750999) (width 0.25) (layer F.Cu) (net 3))
 (segment (start 88.815001 58.490001) (end 91.929003 58.490001) (width 0.25) (layer F.Cu) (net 3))
 (segment (start 92.190001 58.750999) (end 92.190001 72.252821) (width 0.25) (layer F.Cu) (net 3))
 (segment (start 90.603411 73.839411) (end 89.841411 74.601411) (width 0.25) (layer F.Cu) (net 3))
 (segment (start 91.936001 72.506821) (end 90.603411 73.839411) (width 0.25) (layer F.Cu) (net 3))
 (segment (start 89.580003 62.300001) (end 88.815001 62.300001) (width 0.25) (layer F.Cu) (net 5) (status 30))
 (segment (start 86.805002 63.06) (end 87.565001 62.300001) (width 0.25) (layer F.Cu) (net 5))
 (segment (start 87.565001 62.300001) (end 88.815001 62.300001) (width 0.25) (layer F.Cu) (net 5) (status 20))
 (segment (start 85.344 76.454) (end 86.805002 74.992998) (width 0.25) (layer F.Cu) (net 5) (status 10))
 (segment (start 86.805002 74.992998) (end 86.805002 63.06) (width 0.25) (layer F.Cu) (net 5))
 (segment (start 77.955 83.646002) (end 77.955 78.232) (width 0.25) (layer F.Cu) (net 5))
 (segment (start 77.056001 84.545001) (end 77.955 83.646002) (width 0.25) (layer F.Cu) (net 5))
 (segment (start 74.955001 84.545001) (end 77.056001 84.545001) (width 0.25) (layer F.Cu) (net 5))
 (segment (start 74.91 84.5) (end 74.955001 84.545001) (width 0.25) (layer F.Cu) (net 5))
 (segment (start 83.566 78.232) (end 77.955 78.232) (width 0.25) (layer F.Cu) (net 5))
 (segment (start 85.344 76.454) (end 83.566 78.232) (width 0.25) (layer F.Cu) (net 5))
 (segment (start 84.760001 73.460001) (end 84.760001 74.710001) (width 0.25) (layer F.Cu) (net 11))
 (via (at 71.628 78.74) (size 0.8) (drill 0.4) (layers F.Cu B.Cu) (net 11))
 (via (at 72.644 76.2) (size 0.8) (drill 0.4) (layers F.Cu B.Cu) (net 11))
 (segment (start 71.628 79.818) (end 72.105 80.295) (width 0.25) (layer F.Cu) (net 11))
 (segment (start 71.628 78.74) (end 71.628 79.818) (width 0.25) (layer F.Cu) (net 11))
 (segment (start 72.41 80.6) (end 72.105 80.295) (width 0.25) (layer F.Cu) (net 11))
 (segment (start 72.105 80.295) (end 71.882 80.072) (width 0.25) (layer F.Cu) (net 11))
 (segment (start 71.628 77.216) (end 72.644 76.2) (width 0.25) (layer B.Cu) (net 11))
 (segment (start 71.628 78.74) (end 71.628 77.216) (width 0.25) (layer B.Cu) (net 11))
 (segment (start 83.270002 76.2) (end 83.926001 75.544001) (width 0.25) (layer F.Cu) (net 11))
 (segment (start 72.644 76.2) (end 83.270002 76.2) (width 0.25) (layer F.Cu) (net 11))
 (segment (start 84.760001 74.710001) (end 83.926001 75.544001) (width 0.25) (layer F.Cu) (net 11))
 (segment (start 71.753002 57.282) (end 71.815001 57.220001) (width 0.5) (layer F.Cu) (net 4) (status 30))
 (segment (start 71.12 87.63) (end 68.491999 85.001999) (width 0.5) (layer F.Cu) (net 4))
 (segment (start 80.01 87.63) (end 71.12 87.63) (width 0.5) (layer F.Cu) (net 4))
 (segment (start 68.491999 85.001999) (end 68.491999 80.098001) (width 0.5) (layer F.Cu) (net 4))
 (segment (start 70.508001 80.098001) (end 71.60999 81.19999) (width 0.5) (layer F.Cu) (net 4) (status 20))
 (segment (start 68.491999 80.098001) (end 70.508001 80.098001) (width 0.5) (layer F.Cu) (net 4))
 (segment (start 70.612 79.994002) (end 70.508001 80.098001) (width 0.5) (layer F.Cu) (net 4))
 (segment (start 70.612 77.701) (end 70.612 79.994002) (width 0.5) (layer F.Cu) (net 4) (status 10))
 (segment (start 69.652999 57.220001) (end 69.596 57.277) (width 0.5) (layer F.Cu) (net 4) (status 30))
 (segment (start 71.815001 57.220001) (end 69.652999 57.220001) (width 0.5) (layer F.Cu) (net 4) (status 30))
 (segment (start 69.215 57.277) (end 69.596 57.277) (width 0.5) (layer F.Cu) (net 4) (status 30))
 (segment (start 68.491999 58.000001) (end 69.215 57.277) (width 0.5) (layer F.Cu) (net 4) (status 20))
 (segment (start 68.491999 80.098001) (end 68.491999 58.000001) (width 0.5) (layer F.Cu) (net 4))
 (segment (start 86.04 80.96) (end 85.344 80.264) (width 0.5) (layer F.Cu) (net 4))
 (segment (start 87.9 80.96) (end 86.04 80.96) (width 0.5) (layer F.Cu) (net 4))
 (segment (start 86.04 81.6) (end 80.01 87.63) (width 0.5) (layer F.Cu) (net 4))
 (segment (start 86.04 80.96) (end 86.04 81.6) (width 0.5) (layer F.Cu) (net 4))
 (segment (start 75.207 78.232) (end 75.184 78.255) (width 0.25) (layer F.Cu) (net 4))
 (segment (start 76.985 78.232) (end 75.207 78.232) (width 0.5) (layer F.Cu) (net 4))
 (segment (start 72.136 77.216) (end 71.651 77.701) (width 0.5) (layer F.Cu) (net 4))
 (segment (start 71.651 77.701) (end 70.612 77.701) (width 0.5) (layer F.Cu) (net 4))
 (segment (start 74.93 77.216) (end 72.136 77.216) (width 0.5) (layer F.Cu) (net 4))
 (segment (start 75.184 78.255) (end 75.184 77.47) (width 0.5) (layer F.Cu) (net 4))
 (segment (start 75.184 77.47) (end 74.93 77.216) (width 0.5) (layer F.Cu) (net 4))
 (segment (start 84.559 80.264) (end 83.035 81.788) (width 0.5) (layer F.Cu) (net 4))
 (segment (start 85.344 80.264) (end 84.559 80.264) (width 0.5) (layer F.Cu) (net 4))
 (segment (start 74.41 80.6) (end 74.41 80.109298) (width 0.25) (layer F.Cu) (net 6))
 (segment (start 74.41 79.999) (end 74.41 80.6) (width 0.25) (layer F.Cu) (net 6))
 (segment (start 75.184 79.225) (end 74.41 79.999) (width 0.25) (layer F.Cu) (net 6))
 (segment (start 72.91 85.309) (end 72.367 85.852) (width 0.25) (layer F.Cu) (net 9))
 (segment (start 72.91 84.5) (end 72.91 85.309) (width 0.25) (layer F.Cu) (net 9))
 (segment (start 73.429 80.581) (end 73.41 80.6) (width 0.25) (layer F.Cu) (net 7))
 (segment (start 73.41 79.483) (end 73.175 79.248) (width 0.25) (layer F.Cu) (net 7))
 (segment (start 73.41 80.6) (end 73.41 79.483) (width 0.25) (layer F.Cu) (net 7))
 (segment (start 88.885002 59.69) (end 88.815001 59.760001) (width 0.25) (layer F.Cu) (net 2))
 (segment (start 91.115999 59.760001) (end 91.44 59.436) (width 0.25) (layer F.Cu) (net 2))
 (segment (start 88.815001 59.760001) (end 91.115999 59.760001) (width 0.25) (layer F.Cu) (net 2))
 (segment (start 91.002001 61.030001) (end 91.44 61.468) (width 0.25) (layer F.Cu) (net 1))
 (segment (start 88.815001 61.030001) (end 91.002001 61.030001) (width 0.25) (layer F.Cu) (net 1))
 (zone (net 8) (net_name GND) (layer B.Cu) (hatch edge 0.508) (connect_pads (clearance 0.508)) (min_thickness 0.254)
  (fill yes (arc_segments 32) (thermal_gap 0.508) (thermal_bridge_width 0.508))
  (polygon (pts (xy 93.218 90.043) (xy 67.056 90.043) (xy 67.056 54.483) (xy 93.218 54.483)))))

